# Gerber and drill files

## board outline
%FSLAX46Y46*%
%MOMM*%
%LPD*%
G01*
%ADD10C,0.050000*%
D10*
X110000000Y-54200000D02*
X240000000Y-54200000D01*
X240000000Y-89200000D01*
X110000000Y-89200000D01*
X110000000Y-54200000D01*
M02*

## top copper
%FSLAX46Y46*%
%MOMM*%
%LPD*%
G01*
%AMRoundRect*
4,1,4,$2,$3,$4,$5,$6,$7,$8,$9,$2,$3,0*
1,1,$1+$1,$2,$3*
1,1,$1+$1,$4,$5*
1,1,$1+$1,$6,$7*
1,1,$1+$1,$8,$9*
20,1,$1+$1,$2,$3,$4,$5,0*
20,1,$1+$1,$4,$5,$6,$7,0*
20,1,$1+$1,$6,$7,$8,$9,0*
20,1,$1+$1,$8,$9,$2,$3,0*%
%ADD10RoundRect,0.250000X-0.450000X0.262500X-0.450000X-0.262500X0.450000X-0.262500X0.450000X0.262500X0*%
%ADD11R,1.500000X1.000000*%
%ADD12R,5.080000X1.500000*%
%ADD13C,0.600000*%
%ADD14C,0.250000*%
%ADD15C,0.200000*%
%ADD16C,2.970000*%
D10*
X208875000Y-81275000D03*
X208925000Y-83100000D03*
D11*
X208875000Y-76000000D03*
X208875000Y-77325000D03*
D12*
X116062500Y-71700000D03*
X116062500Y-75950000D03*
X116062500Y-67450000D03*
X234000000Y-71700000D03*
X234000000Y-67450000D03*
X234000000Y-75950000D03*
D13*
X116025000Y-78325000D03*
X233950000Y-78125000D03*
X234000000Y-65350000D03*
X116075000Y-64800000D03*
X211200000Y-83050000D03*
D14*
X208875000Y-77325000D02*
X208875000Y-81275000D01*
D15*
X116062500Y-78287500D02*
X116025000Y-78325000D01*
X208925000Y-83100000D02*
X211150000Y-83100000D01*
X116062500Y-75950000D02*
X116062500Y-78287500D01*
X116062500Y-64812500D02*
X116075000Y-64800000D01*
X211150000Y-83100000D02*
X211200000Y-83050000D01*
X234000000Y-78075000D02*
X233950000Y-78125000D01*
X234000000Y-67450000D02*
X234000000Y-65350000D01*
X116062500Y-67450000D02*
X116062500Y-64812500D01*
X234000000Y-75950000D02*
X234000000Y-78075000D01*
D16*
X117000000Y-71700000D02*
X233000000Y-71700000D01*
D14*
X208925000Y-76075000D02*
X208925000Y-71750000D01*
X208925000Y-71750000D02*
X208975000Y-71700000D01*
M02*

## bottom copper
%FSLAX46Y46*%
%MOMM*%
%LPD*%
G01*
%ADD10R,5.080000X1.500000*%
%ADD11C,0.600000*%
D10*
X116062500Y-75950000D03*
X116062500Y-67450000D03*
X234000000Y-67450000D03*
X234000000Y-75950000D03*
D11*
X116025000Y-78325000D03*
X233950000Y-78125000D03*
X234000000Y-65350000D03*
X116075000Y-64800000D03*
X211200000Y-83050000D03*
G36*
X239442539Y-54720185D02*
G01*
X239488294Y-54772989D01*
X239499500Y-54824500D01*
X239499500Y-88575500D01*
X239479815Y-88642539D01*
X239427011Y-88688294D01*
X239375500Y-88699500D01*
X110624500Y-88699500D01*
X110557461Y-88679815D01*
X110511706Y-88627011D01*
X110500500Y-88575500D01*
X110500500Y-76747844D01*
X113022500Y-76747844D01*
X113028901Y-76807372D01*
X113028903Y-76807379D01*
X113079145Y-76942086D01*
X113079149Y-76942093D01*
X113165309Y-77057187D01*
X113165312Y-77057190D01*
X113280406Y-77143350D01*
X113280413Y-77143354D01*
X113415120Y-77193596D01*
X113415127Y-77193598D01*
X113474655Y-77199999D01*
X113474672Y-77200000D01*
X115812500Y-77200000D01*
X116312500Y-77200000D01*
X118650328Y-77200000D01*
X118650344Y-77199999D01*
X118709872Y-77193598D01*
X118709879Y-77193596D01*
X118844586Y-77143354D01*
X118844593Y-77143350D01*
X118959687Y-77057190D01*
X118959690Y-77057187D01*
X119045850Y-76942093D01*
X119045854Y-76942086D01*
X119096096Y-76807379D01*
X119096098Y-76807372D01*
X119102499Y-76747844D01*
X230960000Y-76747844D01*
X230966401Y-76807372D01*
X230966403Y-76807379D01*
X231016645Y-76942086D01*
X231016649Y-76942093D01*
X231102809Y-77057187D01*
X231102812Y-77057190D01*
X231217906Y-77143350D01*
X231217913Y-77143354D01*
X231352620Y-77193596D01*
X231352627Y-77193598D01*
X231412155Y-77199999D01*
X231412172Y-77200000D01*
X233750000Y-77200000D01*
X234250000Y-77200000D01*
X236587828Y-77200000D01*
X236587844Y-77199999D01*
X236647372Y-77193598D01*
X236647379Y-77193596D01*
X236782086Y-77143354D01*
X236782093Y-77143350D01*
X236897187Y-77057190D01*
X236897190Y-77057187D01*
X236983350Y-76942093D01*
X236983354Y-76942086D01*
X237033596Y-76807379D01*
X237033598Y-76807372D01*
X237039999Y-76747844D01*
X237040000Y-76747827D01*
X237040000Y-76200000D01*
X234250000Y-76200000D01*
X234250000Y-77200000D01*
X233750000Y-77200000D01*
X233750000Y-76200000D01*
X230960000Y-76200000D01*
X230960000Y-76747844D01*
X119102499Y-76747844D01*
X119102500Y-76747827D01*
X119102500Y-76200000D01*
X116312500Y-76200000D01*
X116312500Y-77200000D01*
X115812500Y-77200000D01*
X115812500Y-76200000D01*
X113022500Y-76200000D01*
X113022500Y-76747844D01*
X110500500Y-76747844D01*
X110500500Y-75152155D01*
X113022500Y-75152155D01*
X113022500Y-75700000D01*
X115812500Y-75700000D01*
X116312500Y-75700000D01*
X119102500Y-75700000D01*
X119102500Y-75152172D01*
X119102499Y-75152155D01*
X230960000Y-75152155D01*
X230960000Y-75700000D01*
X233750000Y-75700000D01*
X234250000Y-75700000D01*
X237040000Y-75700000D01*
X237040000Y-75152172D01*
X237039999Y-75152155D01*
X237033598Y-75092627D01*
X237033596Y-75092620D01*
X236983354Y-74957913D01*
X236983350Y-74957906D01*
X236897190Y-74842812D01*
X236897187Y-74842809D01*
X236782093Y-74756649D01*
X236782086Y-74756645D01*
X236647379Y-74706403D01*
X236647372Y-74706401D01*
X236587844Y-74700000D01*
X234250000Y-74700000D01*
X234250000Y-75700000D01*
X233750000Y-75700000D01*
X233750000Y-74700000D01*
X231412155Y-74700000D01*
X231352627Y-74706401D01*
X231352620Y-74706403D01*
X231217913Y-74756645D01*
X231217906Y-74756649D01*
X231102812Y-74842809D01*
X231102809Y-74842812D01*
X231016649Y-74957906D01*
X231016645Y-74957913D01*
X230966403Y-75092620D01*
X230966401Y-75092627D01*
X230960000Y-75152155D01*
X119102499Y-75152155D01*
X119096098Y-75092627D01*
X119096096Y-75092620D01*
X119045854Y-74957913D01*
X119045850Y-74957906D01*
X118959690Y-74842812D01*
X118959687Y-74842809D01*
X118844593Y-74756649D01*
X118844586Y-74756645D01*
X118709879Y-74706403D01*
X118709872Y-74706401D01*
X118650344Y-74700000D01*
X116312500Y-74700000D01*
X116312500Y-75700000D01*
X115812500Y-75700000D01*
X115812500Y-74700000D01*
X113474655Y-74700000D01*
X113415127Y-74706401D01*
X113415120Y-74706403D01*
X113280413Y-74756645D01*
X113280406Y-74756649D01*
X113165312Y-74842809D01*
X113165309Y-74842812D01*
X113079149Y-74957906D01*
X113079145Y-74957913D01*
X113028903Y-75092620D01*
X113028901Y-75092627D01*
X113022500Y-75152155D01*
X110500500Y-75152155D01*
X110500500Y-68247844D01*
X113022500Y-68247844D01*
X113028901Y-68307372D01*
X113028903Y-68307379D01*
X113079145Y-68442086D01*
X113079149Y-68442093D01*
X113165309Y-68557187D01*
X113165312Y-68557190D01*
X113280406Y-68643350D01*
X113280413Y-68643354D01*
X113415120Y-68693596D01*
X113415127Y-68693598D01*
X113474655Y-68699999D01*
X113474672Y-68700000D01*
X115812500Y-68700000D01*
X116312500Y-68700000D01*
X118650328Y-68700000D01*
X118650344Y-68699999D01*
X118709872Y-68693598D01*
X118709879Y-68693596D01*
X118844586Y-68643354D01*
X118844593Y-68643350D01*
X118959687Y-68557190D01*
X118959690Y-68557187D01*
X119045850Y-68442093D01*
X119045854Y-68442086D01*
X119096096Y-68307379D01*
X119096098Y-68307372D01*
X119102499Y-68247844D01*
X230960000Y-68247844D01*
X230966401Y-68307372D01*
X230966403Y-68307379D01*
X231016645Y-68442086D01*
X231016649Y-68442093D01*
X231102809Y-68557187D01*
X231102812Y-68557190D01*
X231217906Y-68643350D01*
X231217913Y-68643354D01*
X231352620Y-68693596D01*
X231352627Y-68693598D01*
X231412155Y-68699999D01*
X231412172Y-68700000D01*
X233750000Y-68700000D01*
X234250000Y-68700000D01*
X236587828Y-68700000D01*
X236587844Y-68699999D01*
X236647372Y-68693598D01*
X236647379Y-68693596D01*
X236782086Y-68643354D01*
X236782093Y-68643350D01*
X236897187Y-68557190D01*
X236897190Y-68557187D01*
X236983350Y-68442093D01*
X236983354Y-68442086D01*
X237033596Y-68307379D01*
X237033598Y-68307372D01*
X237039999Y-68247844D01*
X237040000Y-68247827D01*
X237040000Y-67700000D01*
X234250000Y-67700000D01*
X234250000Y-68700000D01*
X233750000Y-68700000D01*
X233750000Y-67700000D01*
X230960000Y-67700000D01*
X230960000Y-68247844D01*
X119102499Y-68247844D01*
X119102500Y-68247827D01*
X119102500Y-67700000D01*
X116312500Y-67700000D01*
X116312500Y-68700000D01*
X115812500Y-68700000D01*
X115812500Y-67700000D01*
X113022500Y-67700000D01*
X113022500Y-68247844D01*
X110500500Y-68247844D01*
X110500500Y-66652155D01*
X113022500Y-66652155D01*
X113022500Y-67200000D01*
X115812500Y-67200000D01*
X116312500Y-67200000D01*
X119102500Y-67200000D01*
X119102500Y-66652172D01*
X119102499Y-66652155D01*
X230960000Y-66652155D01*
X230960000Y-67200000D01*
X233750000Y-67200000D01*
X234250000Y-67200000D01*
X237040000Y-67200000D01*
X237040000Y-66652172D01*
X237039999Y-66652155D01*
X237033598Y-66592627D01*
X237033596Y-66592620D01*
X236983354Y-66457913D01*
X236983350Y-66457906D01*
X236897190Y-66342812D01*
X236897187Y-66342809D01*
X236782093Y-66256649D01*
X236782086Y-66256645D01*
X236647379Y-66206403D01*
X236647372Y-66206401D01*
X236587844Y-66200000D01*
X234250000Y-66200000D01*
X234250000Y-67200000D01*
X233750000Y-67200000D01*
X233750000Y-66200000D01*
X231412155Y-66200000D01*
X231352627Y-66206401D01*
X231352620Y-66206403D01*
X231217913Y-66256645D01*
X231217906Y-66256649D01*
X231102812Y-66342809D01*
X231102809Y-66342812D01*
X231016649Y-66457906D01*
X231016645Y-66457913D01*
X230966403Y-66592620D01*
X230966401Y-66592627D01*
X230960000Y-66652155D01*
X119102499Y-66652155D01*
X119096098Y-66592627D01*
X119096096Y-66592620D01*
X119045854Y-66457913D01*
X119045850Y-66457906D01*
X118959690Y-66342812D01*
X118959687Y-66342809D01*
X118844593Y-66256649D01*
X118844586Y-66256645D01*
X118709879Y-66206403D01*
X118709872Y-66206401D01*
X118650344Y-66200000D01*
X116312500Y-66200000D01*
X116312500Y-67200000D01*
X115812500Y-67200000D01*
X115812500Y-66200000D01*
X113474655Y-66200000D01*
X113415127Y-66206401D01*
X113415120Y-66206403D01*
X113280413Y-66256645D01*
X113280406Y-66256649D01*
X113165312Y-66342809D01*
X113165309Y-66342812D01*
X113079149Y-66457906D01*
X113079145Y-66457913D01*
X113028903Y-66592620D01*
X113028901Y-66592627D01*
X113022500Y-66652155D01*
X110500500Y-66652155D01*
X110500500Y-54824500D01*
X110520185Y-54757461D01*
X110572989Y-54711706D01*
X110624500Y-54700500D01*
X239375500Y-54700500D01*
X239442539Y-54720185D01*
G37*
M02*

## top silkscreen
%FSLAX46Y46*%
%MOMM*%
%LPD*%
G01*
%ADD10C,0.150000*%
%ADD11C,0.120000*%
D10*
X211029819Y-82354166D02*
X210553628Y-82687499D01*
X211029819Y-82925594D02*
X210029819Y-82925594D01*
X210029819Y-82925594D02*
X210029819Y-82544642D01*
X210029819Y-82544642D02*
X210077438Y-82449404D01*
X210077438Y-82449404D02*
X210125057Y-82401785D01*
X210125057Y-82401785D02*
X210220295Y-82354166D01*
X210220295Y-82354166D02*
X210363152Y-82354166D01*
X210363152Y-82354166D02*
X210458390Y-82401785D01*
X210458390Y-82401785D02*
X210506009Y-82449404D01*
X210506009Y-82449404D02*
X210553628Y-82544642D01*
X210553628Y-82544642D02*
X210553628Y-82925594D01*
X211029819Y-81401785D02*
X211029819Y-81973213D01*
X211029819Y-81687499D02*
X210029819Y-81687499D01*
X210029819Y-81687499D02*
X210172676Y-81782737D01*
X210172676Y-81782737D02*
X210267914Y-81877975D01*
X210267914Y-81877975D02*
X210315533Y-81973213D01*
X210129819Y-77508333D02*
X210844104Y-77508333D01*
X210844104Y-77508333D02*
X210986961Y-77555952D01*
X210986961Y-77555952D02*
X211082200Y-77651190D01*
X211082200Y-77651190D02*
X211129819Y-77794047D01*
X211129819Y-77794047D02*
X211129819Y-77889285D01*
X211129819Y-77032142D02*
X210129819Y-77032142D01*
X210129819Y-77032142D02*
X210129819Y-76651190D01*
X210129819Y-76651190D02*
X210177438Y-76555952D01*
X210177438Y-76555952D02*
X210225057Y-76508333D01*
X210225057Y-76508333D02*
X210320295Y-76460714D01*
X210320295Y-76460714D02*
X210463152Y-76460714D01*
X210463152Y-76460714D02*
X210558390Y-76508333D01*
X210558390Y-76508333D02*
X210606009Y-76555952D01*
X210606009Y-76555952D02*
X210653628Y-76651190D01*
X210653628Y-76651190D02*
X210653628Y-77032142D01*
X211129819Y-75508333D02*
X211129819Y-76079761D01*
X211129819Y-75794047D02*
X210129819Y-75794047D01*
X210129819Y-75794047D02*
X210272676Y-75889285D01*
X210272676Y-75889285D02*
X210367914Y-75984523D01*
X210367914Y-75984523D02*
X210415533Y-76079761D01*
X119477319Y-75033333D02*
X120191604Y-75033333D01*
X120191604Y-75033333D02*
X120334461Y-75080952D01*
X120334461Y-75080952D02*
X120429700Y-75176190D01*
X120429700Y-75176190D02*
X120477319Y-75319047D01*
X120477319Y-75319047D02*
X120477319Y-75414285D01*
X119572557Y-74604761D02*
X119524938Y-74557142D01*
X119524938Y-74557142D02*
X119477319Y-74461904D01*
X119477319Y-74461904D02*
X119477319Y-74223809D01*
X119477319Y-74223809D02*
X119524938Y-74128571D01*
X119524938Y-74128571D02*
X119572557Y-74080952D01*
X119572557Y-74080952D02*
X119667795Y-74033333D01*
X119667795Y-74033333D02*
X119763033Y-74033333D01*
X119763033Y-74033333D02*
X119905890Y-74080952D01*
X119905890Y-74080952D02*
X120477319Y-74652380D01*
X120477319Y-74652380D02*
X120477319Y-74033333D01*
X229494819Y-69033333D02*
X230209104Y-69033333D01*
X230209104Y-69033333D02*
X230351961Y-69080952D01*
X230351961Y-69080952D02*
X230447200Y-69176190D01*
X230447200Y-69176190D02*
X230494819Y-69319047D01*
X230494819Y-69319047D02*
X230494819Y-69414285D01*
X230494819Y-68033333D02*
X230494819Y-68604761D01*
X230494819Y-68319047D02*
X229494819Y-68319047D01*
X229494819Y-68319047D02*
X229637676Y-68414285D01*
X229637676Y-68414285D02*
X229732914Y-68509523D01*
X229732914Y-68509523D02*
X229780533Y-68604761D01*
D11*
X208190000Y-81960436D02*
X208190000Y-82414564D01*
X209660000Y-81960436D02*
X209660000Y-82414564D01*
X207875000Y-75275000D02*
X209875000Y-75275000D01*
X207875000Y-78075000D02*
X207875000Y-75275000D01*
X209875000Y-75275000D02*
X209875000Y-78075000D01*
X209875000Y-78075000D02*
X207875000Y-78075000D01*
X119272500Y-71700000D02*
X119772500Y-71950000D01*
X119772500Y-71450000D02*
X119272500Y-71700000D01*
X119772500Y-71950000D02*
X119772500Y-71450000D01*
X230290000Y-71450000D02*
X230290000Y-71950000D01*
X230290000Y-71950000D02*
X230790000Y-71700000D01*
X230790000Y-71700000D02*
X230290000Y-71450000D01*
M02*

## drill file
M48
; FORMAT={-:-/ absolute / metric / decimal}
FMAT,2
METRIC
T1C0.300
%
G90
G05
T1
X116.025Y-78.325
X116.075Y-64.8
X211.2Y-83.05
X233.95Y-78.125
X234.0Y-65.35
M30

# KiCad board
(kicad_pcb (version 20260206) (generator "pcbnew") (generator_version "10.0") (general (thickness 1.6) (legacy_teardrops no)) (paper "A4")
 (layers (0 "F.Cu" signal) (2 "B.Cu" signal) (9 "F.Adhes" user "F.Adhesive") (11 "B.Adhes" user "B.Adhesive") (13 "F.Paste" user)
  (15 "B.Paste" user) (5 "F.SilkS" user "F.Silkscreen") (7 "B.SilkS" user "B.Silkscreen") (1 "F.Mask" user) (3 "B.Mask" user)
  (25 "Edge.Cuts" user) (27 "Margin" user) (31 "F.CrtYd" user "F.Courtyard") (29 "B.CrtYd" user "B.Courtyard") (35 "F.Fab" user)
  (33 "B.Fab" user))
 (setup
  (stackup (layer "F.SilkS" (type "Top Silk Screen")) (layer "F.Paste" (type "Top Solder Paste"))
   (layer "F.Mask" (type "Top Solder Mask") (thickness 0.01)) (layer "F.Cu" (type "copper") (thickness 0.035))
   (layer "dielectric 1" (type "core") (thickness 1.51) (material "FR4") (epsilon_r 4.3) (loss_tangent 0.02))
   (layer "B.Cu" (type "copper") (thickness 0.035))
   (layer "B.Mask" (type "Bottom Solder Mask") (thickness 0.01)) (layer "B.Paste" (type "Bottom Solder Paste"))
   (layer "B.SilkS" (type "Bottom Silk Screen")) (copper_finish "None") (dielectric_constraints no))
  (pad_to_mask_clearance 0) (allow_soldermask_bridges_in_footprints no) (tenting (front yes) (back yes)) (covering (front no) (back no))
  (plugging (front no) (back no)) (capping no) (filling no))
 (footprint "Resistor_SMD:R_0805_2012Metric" (layer "F.Cu") (at 208.925 82.1875 -90)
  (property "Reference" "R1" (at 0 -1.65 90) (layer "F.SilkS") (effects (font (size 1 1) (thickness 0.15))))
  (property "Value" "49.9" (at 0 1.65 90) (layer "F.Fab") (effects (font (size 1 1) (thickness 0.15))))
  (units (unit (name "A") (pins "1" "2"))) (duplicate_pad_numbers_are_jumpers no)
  (fp_line (start -0.227064 0.735) (end 0.227064 0.735) (stroke (width 0.12) (type solid)) (layer "F.SilkS"))
  (fp_line (start -0.227064 -0.735) (end 0.227064 -0.735) (stroke (width 0.12) (type solid)) (layer "F.SilkS"))
  (pad "1" smd roundrect (at -0.9125 0.05 270) (size 1.025 1.4) (layers "F.Cu" "F.Mask" "F.Paste") (roundrect_rratio 0.243902)
   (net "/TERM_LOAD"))
  (pad "2" smd roundrect (at 0.9125 0 270) (size 1.025 1.4) (layers "F.Cu" "F.Mask" "F.Paste") (roundrect_rratio 0.243902) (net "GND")))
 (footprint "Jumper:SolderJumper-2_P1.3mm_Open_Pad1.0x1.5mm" (layer "F.Cu") (at 208.875 76.675 -90)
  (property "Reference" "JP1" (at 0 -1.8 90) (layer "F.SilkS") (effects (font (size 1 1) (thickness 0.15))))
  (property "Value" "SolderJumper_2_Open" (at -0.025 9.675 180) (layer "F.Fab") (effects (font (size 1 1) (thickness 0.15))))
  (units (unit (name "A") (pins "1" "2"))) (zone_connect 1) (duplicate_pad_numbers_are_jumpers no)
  (fp_line (start -1.4 1) (end -1.4 -1) (stroke (width 0.12) (type solid)) (layer "F.SilkS"))
  (fp_line (start 1.4 1) (end -1.4 1) (stroke (width 0.12) (type solid)) (layer "F.SilkS"))
  (fp_line (start -1.4 -1) (end 1.4 -1) (stroke (width 0.12) (type solid)) (layer "F.SilkS"))
  (fp_line (start 1.4 -1) (end 1.4 1) (stroke (width 0.12) (type solid)) (layer "F.SilkS"))
  (pad "1" smd rect (at -0.675 0 270) (size 1 1.5) (layers "F.Cu" "F.Mask") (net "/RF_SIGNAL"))
  (pad "2" smd rect (at 0.65 0 270) (size 1 1.5) (layers "F.Cu" "F.Mask") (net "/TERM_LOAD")))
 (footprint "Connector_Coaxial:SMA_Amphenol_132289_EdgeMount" (layer "F.Cu") (at 116.0625 71.7 180)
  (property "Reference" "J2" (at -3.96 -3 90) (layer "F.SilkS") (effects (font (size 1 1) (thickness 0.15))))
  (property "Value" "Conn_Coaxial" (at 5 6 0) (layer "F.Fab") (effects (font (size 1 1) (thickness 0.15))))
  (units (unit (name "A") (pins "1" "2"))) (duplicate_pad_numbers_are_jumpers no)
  (fp_line (start -3.21 0) (end -3.71 -0.25) (stroke (width 0.12) (type solid)) (layer "F.SilkS"))
  (fp_line (start -3.71 0.25) (end -3.21 0) (stroke (width 0.12) (type solid)) (layer "F.SilkS"))
  (fp_line (start -3.71 -0.25) (end -3.71 0.25) (stroke (width 0.12) (type solid)) (layer "F.SilkS"))
  (pad "1" smd rect (at 0 0 270) (size 1.5 5.08) (layers "F.Cu" "F.Mask" "F.Paste") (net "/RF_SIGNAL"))
  (pad "2" smd rect (at 0 -4.25 270) (size 1.5 5.08) (layers "F.Cu" "F.Mask" "F.Paste") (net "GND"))
  (pad "2" smd rect (at 0 -4.25 270) (size 1.5 5.08) (layers "B.Cu" "B.Mask" "B.Paste") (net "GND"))
  (pad "2" smd rect (at 0 4.25 270) (size 1.5 5.08) (layers "F.Cu" "F.Mask" "F.Paste") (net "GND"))
  (pad "2" smd rect (at 0 4.25 270) (size 1.5 5.08) (layers "B.Cu" "B.Mask" "B.Paste") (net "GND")))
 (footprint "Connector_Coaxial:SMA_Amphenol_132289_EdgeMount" (layer "F.Cu") (at 234 71.7)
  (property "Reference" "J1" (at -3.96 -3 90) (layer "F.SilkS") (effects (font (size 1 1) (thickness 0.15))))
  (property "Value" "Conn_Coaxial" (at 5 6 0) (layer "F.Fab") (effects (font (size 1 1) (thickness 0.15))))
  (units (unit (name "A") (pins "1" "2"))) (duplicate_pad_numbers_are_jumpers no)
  (fp_line (start -3.71 -0.25) (end -3.71 0.25) (stroke (width 0.12) (type solid)) (layer "F.SilkS"))
  (fp_line (start -3.71 0.25) (end -3.21 0) (stroke (width 0.12) (type solid)) (layer "F.SilkS"))
  (fp_line (start -3.21 0) (end -3.71 -0.25) (stroke (width 0.12) (type solid)) (layer "F.SilkS"))
  (pad "1" smd rect (at 0 0 90) (size 1.5 5.08) (layers "F.Cu" "F.Mask" "F.Paste") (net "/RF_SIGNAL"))
  (pad "2" smd rect (at 0 -4.25 90) (size 1.5 5.08) (layers "F.Cu" "F.Mask" "F.Paste") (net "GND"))
  (pad "2" smd rect (at 0 -4.25 90) (size 1.5 5.08) (layers "B.Cu" "B.Mask" "B.Paste") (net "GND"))
  (pad "2" smd rect (at 0 4.25 90) (size 1.5 5.08) (layers "F.Cu" "F.Mask" "F.Paste") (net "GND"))
  (pad "2" smd rect (at 0 4.25 90) (size 1.5 5.08) (layers "B.Cu" "B.Mask" "B.Paste") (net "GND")))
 (gr_rect (start 110 54.2) (end 240 89.2) (stroke (width 0.05) (type solid)) (fill no) (layer "Edge.Cuts"))
 (segment (start 208.875 77.325) (end 208.875 81.275) (width 0.25) (layer "F.Cu") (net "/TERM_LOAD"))
 (segment (start 116.0625 78.2875) (end 116.025 78.325) (width 0.2) (layer "F.Cu") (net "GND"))
 (segment (start 208.925 83.1) (end 211.15 83.1) (width 0.2) (layer "F.Cu") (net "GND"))
 (segment (start 116.0625 75.95) (end 116.0625 78.2875) (width 0.2) (layer "F.Cu") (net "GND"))
 (segment (start 116.0625 64.8125) (end 116.075 64.8) (width 0.2) (layer "F.Cu") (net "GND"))
 (segment (start 211.15 83.1) (end 211.2 83.05) (width 0.2) (layer "F.Cu") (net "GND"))
 (segment (start 234 78.075) (end 233.95 78.125) (width 0.2) (layer "F.Cu") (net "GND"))
 (segment (start 234 67.45) (end 234 65.35) (width 0.2) (layer "F.Cu") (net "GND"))
 (segment (start 116.0625 67.45) (end 116.0625 64.8125) (width 0.2) (layer "F.Cu") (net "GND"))
 (segment (start 234 75.95) (end 234 78.075) (width 0.2) (layer "F.Cu") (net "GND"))
 (via (at 116.025 78.325) (size 0.6) (drill 0.3) (layers "F.Cu" "B.Cu") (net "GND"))
 (via (at 233.95 78.125) (size 0.6) (drill 0.3) (layers "F.Cu" "B.Cu") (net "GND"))
 (via (at 234 65.35) (size 0.6) (drill 0.3) (layers "F.Cu" "B.Cu") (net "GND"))
 (via (at 116.075 64.8) (size 0.6) (drill 0.3) (layers "F.Cu" "B.Cu") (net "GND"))
 (via (at 211.2 83.05) (size 0.6) (drill 0.3) (layers "F.Cu" "B.Cu") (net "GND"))
 (segment (start 117 71.7) (end 233 71.7) (width 2.97) (layer "F.Cu") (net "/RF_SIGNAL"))
 (segment (start 208.925 76.075) (end 208.925 71.75) (width 0.25) (layer "F.Cu") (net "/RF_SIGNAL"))
 (segment (start 208.925 71.75) (end 208.975 71.7) (width 0.25) (layer "F.Cu") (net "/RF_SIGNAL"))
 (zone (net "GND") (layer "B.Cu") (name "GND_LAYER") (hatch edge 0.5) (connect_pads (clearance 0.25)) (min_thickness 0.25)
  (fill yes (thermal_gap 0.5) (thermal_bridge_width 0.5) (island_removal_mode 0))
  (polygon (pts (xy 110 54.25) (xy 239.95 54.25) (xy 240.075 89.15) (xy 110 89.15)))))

